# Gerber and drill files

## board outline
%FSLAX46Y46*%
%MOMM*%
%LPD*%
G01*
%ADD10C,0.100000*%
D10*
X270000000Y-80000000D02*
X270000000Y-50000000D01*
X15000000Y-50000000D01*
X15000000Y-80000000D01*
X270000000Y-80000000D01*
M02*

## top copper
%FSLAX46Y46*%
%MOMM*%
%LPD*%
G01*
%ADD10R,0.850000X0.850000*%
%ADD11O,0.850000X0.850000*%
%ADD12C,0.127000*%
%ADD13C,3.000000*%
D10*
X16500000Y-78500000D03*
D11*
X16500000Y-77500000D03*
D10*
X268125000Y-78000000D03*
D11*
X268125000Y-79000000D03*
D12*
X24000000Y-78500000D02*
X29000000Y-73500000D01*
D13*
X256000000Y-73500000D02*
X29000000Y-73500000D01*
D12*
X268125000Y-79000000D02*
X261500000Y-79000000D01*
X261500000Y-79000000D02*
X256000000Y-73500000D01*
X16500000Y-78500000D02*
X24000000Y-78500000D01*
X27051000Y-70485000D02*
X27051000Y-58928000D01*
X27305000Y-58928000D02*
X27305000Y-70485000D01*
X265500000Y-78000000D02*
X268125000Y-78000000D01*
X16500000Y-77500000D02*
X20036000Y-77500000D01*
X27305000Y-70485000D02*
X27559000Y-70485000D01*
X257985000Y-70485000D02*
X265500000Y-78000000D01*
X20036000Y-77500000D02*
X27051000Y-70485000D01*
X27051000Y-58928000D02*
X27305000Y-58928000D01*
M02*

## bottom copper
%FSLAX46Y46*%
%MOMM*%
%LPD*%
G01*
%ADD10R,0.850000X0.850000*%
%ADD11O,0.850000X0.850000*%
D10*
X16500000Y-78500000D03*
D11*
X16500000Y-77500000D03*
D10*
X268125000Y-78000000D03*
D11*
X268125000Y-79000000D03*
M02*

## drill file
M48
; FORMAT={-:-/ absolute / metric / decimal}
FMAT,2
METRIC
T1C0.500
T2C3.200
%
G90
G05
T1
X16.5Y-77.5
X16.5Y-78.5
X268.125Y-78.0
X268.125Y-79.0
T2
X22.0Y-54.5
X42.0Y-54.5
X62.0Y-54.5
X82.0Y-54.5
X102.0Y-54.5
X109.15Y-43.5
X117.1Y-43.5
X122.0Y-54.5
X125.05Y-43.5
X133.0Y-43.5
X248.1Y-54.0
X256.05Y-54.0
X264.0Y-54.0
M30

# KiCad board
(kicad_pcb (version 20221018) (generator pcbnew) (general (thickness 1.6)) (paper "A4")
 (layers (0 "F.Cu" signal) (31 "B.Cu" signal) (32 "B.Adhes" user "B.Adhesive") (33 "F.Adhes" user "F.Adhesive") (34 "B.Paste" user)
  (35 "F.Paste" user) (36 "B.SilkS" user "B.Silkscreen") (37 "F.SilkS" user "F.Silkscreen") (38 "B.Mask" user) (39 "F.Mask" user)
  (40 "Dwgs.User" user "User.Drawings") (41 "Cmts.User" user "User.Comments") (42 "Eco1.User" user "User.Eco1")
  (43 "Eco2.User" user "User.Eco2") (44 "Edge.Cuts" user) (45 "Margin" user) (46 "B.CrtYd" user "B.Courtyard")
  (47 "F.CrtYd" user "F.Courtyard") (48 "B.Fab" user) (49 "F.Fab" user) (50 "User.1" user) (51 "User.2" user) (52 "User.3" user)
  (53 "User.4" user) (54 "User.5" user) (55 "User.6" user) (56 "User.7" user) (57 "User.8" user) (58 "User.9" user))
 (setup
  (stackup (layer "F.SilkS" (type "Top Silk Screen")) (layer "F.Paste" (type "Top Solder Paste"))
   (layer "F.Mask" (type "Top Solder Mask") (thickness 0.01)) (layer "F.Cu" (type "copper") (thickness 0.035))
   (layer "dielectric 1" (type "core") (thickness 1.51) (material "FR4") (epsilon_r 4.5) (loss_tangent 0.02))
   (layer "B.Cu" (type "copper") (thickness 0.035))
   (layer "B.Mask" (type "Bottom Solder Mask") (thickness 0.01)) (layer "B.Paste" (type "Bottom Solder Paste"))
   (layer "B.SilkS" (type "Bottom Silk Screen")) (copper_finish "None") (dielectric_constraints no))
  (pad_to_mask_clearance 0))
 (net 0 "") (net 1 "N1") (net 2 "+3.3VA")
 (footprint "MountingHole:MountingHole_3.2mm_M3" (layer "F.Cu") (at 256.05 54 90)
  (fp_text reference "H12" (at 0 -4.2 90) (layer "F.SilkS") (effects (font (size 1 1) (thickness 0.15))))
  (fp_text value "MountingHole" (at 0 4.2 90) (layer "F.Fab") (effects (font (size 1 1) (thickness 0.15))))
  (pad "" np_thru_hole circle (at 0 0 90) (size 3.2 3.2) (drill 3.2) (layers "*.Cu" "*.Mask")))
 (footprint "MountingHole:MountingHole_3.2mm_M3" (layer "F.Cu") (at 22 54.5 180)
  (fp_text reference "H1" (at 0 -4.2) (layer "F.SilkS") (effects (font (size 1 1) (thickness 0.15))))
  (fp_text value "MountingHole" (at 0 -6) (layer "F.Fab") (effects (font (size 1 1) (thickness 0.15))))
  (pad "" np_thru_hole circle (at 0 0 180) (size 3.2 3.2) (drill 3.2) (layers "*.Cu" "*.Mask")))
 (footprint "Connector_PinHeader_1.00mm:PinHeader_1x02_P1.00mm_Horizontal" (layer "F.Cu") (at 16.5 78.5 180)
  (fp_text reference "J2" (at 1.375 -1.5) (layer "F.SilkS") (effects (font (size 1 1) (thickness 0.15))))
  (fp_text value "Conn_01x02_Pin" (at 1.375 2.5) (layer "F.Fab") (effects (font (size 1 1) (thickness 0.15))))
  (pad "1" thru_hole rect (at 0 0 180) (size 0.85 0.85) (drill 0.5) (layers "*.Cu" "*.Mask") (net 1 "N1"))
  (pad "2" thru_hole oval (at 0 1 180) (size 0.85 0.85) (drill 0.5) (layers "*.Cu" "*.Mask") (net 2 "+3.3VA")))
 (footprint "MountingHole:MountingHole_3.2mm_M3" (layer "F.Cu") (at 109.15 43.5 90)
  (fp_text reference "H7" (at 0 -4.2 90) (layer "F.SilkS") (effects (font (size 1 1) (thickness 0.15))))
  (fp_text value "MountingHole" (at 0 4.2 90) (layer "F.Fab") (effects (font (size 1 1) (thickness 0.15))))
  (pad "" np_thru_hole circle (at 0 0 90) (size 3.2 3.2) (drill 3.2) (layers "*.Cu" "*.Mask")))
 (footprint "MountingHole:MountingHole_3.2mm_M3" (layer "F.Cu") (at 122 54.5 90)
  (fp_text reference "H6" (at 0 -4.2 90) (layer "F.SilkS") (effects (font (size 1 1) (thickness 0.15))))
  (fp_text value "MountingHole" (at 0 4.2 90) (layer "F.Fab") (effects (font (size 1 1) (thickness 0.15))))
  (pad "" np_thru_hole circle (at 0 0 90) (size 3.2 3.2) (drill 3.2) (layers "*.Cu" "*.Mask")))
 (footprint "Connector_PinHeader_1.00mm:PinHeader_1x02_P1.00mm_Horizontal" (layer "F.Cu") (at 268.125 78)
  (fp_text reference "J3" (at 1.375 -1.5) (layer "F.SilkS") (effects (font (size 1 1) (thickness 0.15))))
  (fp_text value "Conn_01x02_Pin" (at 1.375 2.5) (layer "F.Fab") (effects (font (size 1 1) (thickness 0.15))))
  (pad "1" thru_hole rect (at 0 0) (size 0.85 0.85) (drill 0.5) (layers "*.Cu" "*.Mask") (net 2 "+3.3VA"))
  (pad "2" thru_hole oval (at 0 1) (size 0.85 0.85) (drill 0.5) (layers "*.Cu" "*.Mask") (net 1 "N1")))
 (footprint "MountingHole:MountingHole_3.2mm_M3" (layer "F.Cu") (at 102 54.5 180)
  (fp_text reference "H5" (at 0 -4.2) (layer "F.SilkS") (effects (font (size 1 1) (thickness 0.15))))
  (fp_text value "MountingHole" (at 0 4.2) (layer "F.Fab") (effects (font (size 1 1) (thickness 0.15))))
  (pad "" np_thru_hole circle (at 0 0 180) (size 3.2 3.2) (drill 3.2) (layers "*.Cu" "*.Mask")))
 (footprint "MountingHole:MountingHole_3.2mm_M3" (layer "F.Cu") (at 264 54 90)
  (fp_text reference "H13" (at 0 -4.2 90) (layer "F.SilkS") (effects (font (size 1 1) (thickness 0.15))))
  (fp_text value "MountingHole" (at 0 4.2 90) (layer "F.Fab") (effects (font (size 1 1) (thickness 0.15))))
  (pad "" np_thru_hole circle (at 0 0 90) (size 3.2 3.2) (drill 3.2) (layers "*.Cu" "*.Mask")))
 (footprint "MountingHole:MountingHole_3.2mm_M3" (layer "F.Cu") (at 42 54.5 180)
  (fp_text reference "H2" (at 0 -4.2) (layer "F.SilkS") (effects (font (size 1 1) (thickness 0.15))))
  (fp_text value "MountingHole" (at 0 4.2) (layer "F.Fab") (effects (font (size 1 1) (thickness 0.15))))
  (pad "" np_thru_hole circle (at 0 0 180) (size 3.2 3.2) (drill 3.2) (layers "*.Cu" "*.Mask")))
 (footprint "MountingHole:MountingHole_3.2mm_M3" (layer "F.Cu") (at 125.05 43.5 90)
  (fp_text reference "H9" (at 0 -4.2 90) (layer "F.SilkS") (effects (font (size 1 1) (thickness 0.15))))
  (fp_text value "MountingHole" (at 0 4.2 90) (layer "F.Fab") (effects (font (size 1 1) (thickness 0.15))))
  (pad "" np_thru_hole circle (at 0 0 90) (size 3.2 3.2) (drill 3.2) (layers "*.Cu" "*.Mask")))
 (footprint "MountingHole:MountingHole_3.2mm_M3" (layer "F.Cu") (at 62 54.5 180)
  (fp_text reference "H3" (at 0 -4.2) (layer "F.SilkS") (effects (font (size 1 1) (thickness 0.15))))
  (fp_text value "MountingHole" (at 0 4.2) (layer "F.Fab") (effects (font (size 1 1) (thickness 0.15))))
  (pad "" np_thru_hole circle (at 0 0 180) (size 3.2 3.2) (drill 3.2) (layers "*.Cu" "*.Mask")))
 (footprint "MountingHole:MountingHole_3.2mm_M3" (layer "F.Cu") (at 82 54.5 180)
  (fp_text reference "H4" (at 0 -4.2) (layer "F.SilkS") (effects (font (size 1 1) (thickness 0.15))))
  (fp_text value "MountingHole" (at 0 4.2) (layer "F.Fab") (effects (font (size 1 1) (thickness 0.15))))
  (pad "" np_thru_hole circle (at 0 0 180) (size 3.2 3.2) (drill 3.2) (layers "*.Cu" "*.Mask")))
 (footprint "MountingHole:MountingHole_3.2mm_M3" (layer "F.Cu") (at 248.1 54 90)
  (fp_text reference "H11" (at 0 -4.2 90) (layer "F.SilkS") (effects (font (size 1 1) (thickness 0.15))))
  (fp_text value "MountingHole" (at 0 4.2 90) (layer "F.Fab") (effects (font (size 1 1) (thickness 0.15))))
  (pad "" np_thru_hole circle (at 0 0 90) (size 3.2 3.2) (drill 3.2) (layers "*.Cu" "*.Mask")))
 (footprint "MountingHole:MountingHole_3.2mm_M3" (layer "F.Cu") (at 117.1 43.5 90)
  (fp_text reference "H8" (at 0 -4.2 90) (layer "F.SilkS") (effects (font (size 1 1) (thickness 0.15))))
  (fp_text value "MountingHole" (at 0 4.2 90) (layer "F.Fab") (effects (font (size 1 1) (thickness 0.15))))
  (pad "" np_thru_hole circle (at 0 0 90) (size 3.2 3.2) (drill 3.2) (layers "*.Cu" "*.Mask")))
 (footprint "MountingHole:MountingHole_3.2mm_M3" (layer "F.Cu") (at 133 43.5 90)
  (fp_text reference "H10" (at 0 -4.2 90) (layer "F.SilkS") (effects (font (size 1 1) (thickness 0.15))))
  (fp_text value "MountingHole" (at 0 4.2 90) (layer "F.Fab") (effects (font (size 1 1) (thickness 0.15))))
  (pad "" np_thru_hole circle (at 0 0 90) (size 3.2 3.2) (drill 3.2) (layers "*.Cu" "*.Mask")))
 (gr_poly (pts (xy 270 80) (xy 270 50) (xy 15 50) (xy 15 80)) (stroke (width 0.1) (type solid)) (fill none) (layer "Edge.Cuts"))
 (segment (start 24 78.5) (end 29 73.5) (width 0.127) (layer "F.Cu") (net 1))
 (segment (start 256 73.5) (end 29 73.5) (width 3) (layer "F.Cu") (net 1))
 (segment (start 268.125 79) (end 261.5 79) (width 0.127) (layer "F.Cu") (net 1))
 (segment (start 261.5 79) (end 256 73.5) (width 0.127) (layer "F.Cu") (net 1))
 (segment (start 16.5 78.5) (end 24 78.5) (width 0.127) (layer "F.Cu") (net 1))
 (segment (start 27.051 70.485) (end 27.051 58.928) (width 0.127) (layer "F.Cu") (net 2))
 (segment (start 27.305 58.928) (end 27.305 70.485) (width 0.127) (layer "F.Cu") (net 2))
 (segment (start 265.5 78) (end 268.125 78) (width 0.127) (layer "F.Cu") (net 2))
 (segment (start 16.5 77.5) (end 20.036 77.5) (width 0.127) (layer "F.Cu") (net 2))
 (segment (start 27.305 70.485) (end 27.559 70.485) (width 0.127) (layer "F.Cu") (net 2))
 (segment (start 257.985 70.485) (end 265.5 78) (width 0.127) (layer "F.Cu") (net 2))
 (segment (start 20.036 77.5) (end 27.051 70.485) (width 0.127) (layer "F.Cu") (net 2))
 (segment (start 27.051 58.928) (end 27.305 58.928) (width 0.127) (layer "F.Cu") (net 2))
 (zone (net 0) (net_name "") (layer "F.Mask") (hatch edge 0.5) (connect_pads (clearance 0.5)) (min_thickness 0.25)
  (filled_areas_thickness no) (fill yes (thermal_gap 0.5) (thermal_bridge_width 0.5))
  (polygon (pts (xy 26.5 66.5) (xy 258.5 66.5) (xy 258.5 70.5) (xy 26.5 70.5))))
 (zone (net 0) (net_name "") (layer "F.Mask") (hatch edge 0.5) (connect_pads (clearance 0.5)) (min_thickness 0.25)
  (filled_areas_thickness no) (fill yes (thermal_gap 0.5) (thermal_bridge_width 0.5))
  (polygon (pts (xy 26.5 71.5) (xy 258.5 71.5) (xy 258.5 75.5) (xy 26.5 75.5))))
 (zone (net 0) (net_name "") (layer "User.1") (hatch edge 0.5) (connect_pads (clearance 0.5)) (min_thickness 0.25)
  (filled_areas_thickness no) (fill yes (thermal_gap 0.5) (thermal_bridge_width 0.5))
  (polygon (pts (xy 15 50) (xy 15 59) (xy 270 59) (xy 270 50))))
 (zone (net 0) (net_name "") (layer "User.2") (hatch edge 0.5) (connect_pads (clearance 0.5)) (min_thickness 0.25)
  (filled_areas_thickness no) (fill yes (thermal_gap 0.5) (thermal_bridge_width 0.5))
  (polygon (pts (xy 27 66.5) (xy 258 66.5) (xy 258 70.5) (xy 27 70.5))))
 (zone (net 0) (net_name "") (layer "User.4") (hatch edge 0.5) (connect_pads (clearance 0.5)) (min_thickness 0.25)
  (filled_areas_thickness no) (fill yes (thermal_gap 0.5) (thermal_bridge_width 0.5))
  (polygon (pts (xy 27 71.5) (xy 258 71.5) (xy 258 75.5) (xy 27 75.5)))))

